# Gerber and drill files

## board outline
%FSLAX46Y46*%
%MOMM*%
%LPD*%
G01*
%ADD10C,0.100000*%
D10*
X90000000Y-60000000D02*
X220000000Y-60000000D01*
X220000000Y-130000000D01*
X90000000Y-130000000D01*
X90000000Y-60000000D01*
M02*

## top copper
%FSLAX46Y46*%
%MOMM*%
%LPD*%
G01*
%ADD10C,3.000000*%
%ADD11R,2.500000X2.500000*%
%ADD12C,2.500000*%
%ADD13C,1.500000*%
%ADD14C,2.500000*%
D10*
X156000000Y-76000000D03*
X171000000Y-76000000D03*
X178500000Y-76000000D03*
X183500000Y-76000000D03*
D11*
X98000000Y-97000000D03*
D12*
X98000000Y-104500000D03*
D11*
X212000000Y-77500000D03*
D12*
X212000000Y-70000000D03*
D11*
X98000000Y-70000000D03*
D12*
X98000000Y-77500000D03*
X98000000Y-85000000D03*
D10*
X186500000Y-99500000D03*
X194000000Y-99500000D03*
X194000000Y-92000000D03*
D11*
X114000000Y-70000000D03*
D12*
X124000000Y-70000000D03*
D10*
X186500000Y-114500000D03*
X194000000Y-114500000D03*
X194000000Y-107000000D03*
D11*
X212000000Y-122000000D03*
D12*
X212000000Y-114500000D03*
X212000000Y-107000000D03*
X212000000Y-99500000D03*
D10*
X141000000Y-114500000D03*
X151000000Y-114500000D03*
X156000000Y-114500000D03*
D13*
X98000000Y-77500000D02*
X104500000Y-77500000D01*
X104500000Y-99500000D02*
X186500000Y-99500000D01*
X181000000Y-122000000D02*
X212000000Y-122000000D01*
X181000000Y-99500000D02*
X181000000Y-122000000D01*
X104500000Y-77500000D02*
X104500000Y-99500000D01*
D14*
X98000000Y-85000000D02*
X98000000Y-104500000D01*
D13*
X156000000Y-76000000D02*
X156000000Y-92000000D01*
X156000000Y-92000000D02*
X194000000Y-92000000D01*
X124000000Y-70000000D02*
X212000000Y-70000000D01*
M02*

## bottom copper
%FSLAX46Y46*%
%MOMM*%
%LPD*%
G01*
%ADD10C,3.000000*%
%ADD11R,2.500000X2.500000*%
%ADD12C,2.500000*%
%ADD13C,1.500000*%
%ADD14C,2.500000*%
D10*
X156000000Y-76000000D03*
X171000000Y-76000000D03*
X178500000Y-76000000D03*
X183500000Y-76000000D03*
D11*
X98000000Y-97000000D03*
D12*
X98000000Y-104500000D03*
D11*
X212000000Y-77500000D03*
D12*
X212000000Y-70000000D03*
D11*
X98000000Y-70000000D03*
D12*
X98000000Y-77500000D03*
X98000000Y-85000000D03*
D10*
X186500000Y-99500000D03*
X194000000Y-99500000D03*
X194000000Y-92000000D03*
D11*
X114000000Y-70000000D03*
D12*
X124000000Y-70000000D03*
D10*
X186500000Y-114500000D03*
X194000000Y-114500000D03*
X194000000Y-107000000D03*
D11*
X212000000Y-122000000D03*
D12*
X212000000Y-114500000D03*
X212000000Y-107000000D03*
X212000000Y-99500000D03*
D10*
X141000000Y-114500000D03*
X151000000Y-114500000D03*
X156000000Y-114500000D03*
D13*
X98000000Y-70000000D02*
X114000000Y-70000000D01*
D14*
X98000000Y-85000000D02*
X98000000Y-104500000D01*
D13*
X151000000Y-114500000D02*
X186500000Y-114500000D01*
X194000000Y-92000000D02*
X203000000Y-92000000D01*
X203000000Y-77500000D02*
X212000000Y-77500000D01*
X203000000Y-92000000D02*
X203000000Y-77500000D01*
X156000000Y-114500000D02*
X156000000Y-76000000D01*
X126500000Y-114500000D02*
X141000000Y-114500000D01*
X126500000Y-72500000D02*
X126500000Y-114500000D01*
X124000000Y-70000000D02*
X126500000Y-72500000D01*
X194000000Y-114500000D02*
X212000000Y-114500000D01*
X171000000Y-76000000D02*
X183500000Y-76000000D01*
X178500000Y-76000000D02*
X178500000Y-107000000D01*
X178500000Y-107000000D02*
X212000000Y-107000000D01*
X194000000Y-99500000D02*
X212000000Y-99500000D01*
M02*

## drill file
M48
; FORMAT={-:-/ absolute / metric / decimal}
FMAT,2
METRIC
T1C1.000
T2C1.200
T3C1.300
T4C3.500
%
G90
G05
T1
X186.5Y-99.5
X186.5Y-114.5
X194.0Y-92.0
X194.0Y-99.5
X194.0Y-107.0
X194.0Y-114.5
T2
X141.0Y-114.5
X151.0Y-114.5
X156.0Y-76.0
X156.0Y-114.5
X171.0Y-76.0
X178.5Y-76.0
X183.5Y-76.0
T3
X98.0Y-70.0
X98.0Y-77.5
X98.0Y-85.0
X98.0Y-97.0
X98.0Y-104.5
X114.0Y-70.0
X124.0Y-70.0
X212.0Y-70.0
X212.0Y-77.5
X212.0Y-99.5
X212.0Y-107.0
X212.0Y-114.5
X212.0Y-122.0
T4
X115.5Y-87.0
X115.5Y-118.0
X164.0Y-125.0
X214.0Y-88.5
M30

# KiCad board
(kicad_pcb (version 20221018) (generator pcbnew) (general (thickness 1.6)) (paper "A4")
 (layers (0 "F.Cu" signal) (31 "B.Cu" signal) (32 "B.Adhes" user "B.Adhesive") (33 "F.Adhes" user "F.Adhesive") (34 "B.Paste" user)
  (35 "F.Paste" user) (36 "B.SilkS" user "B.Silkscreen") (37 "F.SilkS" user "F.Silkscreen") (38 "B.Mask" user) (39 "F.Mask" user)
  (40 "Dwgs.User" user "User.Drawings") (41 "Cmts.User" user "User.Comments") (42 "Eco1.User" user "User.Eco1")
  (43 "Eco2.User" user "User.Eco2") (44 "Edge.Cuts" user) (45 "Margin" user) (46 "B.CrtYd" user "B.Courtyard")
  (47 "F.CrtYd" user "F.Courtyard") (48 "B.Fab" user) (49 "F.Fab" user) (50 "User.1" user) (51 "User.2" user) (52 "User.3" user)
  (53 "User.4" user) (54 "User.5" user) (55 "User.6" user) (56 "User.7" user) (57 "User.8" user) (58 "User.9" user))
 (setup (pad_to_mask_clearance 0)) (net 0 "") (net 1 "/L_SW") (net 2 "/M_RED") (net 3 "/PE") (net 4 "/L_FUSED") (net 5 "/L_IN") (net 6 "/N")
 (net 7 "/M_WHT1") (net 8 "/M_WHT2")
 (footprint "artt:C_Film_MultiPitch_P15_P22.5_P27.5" (layer "F.Cu") (at 156 76)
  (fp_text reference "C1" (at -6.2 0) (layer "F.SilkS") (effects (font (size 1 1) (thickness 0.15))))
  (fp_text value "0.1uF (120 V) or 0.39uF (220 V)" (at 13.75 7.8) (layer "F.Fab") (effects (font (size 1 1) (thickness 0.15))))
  (pad "1" thru_hole circle (at 0 0) (size 3 3) (drill 1.2) (layers "*.Cu" "*.Mask") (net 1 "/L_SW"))
  (pad "2" thru_hole circle (at 15 0) (size 3 3) (drill 1.2) (layers "*.Cu" "*.Mask") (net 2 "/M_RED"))
  (pad "2" thru_hole circle (at 22.5 0) (size 3 3) (drill 1.2) (layers "*.Cu" "*.Mask") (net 2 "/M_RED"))
  (pad "2" thru_hole circle (at 27.5 0) (size 3 3) (drill 1.2) (layers "*.Cu" "*.Mask") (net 2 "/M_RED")))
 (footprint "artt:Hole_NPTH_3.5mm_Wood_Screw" (layer "F.Cu") (at 115.5 118)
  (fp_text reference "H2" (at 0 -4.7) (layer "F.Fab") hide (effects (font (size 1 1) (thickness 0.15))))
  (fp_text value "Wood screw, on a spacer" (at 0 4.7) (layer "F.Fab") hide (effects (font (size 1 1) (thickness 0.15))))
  (pad "" np_thru_hole circle (at 0 0) (size 3.5 3.5) (drill 3.5) (layers "*.Cu" "*.Mask")))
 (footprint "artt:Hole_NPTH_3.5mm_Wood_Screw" (layer "F.Cu") (at 115.5 87)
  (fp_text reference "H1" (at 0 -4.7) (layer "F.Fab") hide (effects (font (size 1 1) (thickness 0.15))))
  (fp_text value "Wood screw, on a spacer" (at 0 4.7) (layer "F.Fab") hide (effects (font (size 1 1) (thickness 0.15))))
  (pad "" np_thru_hole circle (at 0 0) (size 3.5 3.5) (drill 3.5) (layers "*.Cu" "*.Mask")))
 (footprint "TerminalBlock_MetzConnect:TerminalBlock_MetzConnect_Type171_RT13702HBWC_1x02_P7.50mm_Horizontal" (layer "F.Cu") (at 98 97 -90)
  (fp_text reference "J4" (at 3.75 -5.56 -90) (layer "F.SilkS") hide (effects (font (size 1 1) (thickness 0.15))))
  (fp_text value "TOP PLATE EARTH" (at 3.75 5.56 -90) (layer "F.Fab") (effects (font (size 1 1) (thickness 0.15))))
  (pad "1" thru_hole rect (at 0 0 270) (size 2.5 2.5) (drill 1.3) (layers "*.Cu" "*.Mask") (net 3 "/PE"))
  (pad "2" thru_hole circle (at 7.5 0 270) (size 2.5 2.5) (drill 1.3) (layers "*.Cu" "*.Mask") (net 3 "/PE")))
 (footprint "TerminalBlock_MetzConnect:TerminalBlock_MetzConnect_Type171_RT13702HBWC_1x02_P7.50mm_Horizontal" (layer "F.Cu")
  (at 212 77.5 90)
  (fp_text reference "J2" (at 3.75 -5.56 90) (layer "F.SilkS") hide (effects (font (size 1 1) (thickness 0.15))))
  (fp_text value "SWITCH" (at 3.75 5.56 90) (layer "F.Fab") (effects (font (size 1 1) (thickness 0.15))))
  (pad "1" thru_hole rect (at 0 0 90) (size 2.5 2.5) (drill 1.3) (layers "*.Cu" "*.Mask") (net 1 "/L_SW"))
  (pad "2" thru_hole circle (at 7.5 0 90) (size 2.5 2.5) (drill 1.3) (layers "*.Cu" "*.Mask") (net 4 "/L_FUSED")))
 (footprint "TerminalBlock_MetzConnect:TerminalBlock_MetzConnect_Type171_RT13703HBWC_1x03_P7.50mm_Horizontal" (layer "F.Cu") (at 98 70 -90)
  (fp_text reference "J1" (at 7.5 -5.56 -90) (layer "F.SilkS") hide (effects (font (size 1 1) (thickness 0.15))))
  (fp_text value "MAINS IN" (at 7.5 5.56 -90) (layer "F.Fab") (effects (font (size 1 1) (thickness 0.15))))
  (pad "1" thru_hole rect (at 0 0 270) (size 2.5 2.5) (drill 1.3) (layers "*.Cu" "*.Mask") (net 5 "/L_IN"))
  (pad "2" thru_hole circle (at 7.5 0 270) (size 2.5 2.5) (drill 1.3) (layers "*.Cu" "*.Mask") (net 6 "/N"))
  (pad "3" thru_hole circle (at 15 0 270) (size 2.5 2.5) (drill 1.3) (layers "*.Cu" "*.Mask") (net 3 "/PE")))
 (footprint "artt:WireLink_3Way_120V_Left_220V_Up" (layer "F.Cu") (at 194 99.5)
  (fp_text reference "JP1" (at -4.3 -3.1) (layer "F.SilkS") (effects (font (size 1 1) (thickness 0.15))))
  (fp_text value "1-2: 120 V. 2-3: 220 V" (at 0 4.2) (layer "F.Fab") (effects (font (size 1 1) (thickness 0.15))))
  (pad "1" thru_hole circle (at -7.5 0) (size 3 3) (drill 1) (layers "*.Cu" "*.Mask") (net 6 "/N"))
  (pad "2" thru_hole circle (at 0 0) (size 3 3) (drill 1) (layers "*.Cu" "*.Mask") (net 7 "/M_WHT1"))
  (pad "3" thru_hole circle (at 0 -7.5) (size 3 3) (drill 1) (layers "*.Cu" "*.Mask") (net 1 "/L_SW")))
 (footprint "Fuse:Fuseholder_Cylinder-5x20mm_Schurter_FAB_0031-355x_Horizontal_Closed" (layer "F.Cu") (at 114 70)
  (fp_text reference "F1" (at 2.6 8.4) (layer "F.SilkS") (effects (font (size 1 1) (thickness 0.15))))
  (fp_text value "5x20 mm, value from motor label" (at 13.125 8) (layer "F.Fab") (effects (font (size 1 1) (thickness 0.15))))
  (pad "1" thru_hole rect (at 0 0) (size 2.5 2.5) (drill 1.3) (layers "*.Cu" "*.Mask") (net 5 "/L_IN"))
  (pad "2" thru_hole circle (at 10 0) (size 2.5 2.5) (drill 1.3) (layers "*.Cu" "*.Mask") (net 4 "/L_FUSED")))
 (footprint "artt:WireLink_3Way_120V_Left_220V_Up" (layer "F.Cu") (at 194 114.5)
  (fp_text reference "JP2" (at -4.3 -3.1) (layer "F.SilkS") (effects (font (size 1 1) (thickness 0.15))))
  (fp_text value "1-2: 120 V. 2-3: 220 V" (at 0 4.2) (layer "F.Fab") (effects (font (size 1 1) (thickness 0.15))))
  (pad "1" thru_hole circle (at -7.5 0) (size 3 3) (drill 1) (layers "*.Cu" "*.Mask") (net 1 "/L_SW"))
  (pad "2" thru_hole circle (at 0 0) (size 3 3) (drill 1) (layers "*.Cu" "*.Mask") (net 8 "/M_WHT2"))
  (pad "3" thru_hole circle (at 0 -7.5) (size 3 3) (drill 1) (layers "*.Cu" "*.Mask") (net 2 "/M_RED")))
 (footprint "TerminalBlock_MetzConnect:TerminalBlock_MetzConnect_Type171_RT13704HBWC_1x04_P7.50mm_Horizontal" (layer "F.Cu") (at 212 122 90)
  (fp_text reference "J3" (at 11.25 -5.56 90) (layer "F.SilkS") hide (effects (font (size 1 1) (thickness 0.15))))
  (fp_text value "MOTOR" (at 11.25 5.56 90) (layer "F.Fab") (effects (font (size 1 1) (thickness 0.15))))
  (pad "1" thru_hole rect (at 0 0 90) (size 2.5 2.5) (drill 1.3) (layers "*.Cu" "*.Mask") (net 6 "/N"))
  (pad "2" thru_hole circle (at 7.5 0 90) (size 2.5 2.5) (drill 1.3) (layers "*.Cu" "*.Mask") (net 8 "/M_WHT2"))
  (pad "3" thru_hole circle (at 15 0 90) (size 2.5 2.5) (drill 1.3) (layers "*.Cu" "*.Mask") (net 2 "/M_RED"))
  (pad "4" thru_hole circle (at 22.5 0 90) (size 2.5 2.5) (drill 1.3) (layers "*.Cu" "*.Mask") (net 7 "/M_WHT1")))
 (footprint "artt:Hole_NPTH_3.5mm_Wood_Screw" (layer "F.Cu") (at 164 125)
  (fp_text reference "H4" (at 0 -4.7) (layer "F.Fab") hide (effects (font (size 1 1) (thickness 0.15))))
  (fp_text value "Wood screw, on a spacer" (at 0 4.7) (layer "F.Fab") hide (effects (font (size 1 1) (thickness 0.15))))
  (pad "" np_thru_hole circle (at 0 0) (size 3.5 3.5) (drill 3.5) (layers "*.Cu" "*.Mask")))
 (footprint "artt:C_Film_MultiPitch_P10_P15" (layer "F.Cu") (at 141 114.5)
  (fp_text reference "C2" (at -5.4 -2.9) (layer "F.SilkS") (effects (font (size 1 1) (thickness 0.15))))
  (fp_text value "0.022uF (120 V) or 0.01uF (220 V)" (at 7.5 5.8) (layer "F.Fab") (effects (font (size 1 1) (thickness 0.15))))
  (pad "1" thru_hole circle (at 0 0) (size 3 3) (drill 1.2) (layers "*.Cu" "*.Mask") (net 4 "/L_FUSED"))
  (pad "2" thru_hole circle (at 10 0) (size 3 3) (drill 1.2) (layers "*.Cu" "*.Mask") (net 1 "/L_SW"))
  (pad "2" thru_hole circle (at 15 0) (size 3 3) (drill 1.2) (layers "*.Cu" "*.Mask") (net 1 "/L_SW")))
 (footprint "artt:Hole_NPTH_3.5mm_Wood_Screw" (layer "F.Cu") (at 214 88.5)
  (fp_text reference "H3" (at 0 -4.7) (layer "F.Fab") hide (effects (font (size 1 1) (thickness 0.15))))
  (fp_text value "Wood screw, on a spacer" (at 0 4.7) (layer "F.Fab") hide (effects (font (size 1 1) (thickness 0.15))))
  (pad "" np_thru_hole circle (at 0 0) (size 3.5 3.5) (drill 3.5) (layers "*.Cu" "*.Mask")))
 (gr_rect (start 90 60) (end 220 130) (stroke (width 0.1) (type default)) (fill none) (layer "Edge.Cuts"))
 (segment (start 98 70) (end 114 70) (width 1.5) (layer "B.Cu") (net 5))
 (segment (start 98 77.5) (end 104.5 77.5) (width 1.5) (layer "F.Cu") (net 6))
 (segment (start 104.5 99.5) (end 186.5 99.5) (width 1.5) (layer "F.Cu") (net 6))
 (segment (start 181 122) (end 212 122) (width 1.5) (layer "F.Cu") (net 6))
 (segment (start 181 99.5) (end 181 122) (width 1.5) (layer "F.Cu") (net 6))
 (segment (start 104.5 77.5) (end 104.5 99.5) (width 1.5) (layer "F.Cu") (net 6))
 (segment (start 98 85) (end 98 104.5) (width 2.5) (layer "F.Cu") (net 3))
 (segment (start 98 85) (end 98 104.5) (width 2.5) (layer "B.Cu") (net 3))
 (segment (start 156 76) (end 156 92) (width 1.5) (layer "F.Cu") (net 1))
 (segment (start 156 92) (end 194 92) (width 1.5) (layer "F.Cu") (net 1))
 (segment (start 151 114.5) (end 186.5 114.5) (width 1.5) (layer "B.Cu") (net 1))
 (segment (start 194 92) (end 203 92) (width 1.5) (layer "B.Cu") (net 1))
 (segment (start 203 77.5) (end 212 77.5) (width 1.5) (layer "B.Cu") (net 1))
 (segment (start 203 92) (end 203 77.5) (width 1.5) (layer "B.Cu") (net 1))
 (segment (start 156 114.5) (end 156 76) (width 1.5) (layer "B.Cu") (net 1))
 (segment (start 124 70) (end 212 70) (width 1.5) (layer "F.Cu") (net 4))
 (segment (start 126.5 114.5) (end 141 114.5) (width 1.5) (layer "B.Cu") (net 4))
 (segment (start 126.5 72.5) (end 126.5 114.5) (width 1.5) (layer "B.Cu") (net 4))
 (segment (start 124 70) (end 126.5 72.5) (width 1.5) (layer "B.Cu") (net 4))
 (segment (start 194 114.5) (end 212 114.5) (width 1.5) (layer "B.Cu") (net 8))
 (segment (start 171 76) (end 183.5 76) (width 1.5) (layer "B.Cu") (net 2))
 (segment (start 178.5 76) (end 178.5 107) (width 1.5) (layer "B.Cu") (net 2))
 (segment (start 178.5 107) (end 212 107) (width 1.5) (layer "B.Cu") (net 2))
 (segment (start 194 99.5) (end 212 99.5) (width 1.5) (layer "B.Cu") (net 7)))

